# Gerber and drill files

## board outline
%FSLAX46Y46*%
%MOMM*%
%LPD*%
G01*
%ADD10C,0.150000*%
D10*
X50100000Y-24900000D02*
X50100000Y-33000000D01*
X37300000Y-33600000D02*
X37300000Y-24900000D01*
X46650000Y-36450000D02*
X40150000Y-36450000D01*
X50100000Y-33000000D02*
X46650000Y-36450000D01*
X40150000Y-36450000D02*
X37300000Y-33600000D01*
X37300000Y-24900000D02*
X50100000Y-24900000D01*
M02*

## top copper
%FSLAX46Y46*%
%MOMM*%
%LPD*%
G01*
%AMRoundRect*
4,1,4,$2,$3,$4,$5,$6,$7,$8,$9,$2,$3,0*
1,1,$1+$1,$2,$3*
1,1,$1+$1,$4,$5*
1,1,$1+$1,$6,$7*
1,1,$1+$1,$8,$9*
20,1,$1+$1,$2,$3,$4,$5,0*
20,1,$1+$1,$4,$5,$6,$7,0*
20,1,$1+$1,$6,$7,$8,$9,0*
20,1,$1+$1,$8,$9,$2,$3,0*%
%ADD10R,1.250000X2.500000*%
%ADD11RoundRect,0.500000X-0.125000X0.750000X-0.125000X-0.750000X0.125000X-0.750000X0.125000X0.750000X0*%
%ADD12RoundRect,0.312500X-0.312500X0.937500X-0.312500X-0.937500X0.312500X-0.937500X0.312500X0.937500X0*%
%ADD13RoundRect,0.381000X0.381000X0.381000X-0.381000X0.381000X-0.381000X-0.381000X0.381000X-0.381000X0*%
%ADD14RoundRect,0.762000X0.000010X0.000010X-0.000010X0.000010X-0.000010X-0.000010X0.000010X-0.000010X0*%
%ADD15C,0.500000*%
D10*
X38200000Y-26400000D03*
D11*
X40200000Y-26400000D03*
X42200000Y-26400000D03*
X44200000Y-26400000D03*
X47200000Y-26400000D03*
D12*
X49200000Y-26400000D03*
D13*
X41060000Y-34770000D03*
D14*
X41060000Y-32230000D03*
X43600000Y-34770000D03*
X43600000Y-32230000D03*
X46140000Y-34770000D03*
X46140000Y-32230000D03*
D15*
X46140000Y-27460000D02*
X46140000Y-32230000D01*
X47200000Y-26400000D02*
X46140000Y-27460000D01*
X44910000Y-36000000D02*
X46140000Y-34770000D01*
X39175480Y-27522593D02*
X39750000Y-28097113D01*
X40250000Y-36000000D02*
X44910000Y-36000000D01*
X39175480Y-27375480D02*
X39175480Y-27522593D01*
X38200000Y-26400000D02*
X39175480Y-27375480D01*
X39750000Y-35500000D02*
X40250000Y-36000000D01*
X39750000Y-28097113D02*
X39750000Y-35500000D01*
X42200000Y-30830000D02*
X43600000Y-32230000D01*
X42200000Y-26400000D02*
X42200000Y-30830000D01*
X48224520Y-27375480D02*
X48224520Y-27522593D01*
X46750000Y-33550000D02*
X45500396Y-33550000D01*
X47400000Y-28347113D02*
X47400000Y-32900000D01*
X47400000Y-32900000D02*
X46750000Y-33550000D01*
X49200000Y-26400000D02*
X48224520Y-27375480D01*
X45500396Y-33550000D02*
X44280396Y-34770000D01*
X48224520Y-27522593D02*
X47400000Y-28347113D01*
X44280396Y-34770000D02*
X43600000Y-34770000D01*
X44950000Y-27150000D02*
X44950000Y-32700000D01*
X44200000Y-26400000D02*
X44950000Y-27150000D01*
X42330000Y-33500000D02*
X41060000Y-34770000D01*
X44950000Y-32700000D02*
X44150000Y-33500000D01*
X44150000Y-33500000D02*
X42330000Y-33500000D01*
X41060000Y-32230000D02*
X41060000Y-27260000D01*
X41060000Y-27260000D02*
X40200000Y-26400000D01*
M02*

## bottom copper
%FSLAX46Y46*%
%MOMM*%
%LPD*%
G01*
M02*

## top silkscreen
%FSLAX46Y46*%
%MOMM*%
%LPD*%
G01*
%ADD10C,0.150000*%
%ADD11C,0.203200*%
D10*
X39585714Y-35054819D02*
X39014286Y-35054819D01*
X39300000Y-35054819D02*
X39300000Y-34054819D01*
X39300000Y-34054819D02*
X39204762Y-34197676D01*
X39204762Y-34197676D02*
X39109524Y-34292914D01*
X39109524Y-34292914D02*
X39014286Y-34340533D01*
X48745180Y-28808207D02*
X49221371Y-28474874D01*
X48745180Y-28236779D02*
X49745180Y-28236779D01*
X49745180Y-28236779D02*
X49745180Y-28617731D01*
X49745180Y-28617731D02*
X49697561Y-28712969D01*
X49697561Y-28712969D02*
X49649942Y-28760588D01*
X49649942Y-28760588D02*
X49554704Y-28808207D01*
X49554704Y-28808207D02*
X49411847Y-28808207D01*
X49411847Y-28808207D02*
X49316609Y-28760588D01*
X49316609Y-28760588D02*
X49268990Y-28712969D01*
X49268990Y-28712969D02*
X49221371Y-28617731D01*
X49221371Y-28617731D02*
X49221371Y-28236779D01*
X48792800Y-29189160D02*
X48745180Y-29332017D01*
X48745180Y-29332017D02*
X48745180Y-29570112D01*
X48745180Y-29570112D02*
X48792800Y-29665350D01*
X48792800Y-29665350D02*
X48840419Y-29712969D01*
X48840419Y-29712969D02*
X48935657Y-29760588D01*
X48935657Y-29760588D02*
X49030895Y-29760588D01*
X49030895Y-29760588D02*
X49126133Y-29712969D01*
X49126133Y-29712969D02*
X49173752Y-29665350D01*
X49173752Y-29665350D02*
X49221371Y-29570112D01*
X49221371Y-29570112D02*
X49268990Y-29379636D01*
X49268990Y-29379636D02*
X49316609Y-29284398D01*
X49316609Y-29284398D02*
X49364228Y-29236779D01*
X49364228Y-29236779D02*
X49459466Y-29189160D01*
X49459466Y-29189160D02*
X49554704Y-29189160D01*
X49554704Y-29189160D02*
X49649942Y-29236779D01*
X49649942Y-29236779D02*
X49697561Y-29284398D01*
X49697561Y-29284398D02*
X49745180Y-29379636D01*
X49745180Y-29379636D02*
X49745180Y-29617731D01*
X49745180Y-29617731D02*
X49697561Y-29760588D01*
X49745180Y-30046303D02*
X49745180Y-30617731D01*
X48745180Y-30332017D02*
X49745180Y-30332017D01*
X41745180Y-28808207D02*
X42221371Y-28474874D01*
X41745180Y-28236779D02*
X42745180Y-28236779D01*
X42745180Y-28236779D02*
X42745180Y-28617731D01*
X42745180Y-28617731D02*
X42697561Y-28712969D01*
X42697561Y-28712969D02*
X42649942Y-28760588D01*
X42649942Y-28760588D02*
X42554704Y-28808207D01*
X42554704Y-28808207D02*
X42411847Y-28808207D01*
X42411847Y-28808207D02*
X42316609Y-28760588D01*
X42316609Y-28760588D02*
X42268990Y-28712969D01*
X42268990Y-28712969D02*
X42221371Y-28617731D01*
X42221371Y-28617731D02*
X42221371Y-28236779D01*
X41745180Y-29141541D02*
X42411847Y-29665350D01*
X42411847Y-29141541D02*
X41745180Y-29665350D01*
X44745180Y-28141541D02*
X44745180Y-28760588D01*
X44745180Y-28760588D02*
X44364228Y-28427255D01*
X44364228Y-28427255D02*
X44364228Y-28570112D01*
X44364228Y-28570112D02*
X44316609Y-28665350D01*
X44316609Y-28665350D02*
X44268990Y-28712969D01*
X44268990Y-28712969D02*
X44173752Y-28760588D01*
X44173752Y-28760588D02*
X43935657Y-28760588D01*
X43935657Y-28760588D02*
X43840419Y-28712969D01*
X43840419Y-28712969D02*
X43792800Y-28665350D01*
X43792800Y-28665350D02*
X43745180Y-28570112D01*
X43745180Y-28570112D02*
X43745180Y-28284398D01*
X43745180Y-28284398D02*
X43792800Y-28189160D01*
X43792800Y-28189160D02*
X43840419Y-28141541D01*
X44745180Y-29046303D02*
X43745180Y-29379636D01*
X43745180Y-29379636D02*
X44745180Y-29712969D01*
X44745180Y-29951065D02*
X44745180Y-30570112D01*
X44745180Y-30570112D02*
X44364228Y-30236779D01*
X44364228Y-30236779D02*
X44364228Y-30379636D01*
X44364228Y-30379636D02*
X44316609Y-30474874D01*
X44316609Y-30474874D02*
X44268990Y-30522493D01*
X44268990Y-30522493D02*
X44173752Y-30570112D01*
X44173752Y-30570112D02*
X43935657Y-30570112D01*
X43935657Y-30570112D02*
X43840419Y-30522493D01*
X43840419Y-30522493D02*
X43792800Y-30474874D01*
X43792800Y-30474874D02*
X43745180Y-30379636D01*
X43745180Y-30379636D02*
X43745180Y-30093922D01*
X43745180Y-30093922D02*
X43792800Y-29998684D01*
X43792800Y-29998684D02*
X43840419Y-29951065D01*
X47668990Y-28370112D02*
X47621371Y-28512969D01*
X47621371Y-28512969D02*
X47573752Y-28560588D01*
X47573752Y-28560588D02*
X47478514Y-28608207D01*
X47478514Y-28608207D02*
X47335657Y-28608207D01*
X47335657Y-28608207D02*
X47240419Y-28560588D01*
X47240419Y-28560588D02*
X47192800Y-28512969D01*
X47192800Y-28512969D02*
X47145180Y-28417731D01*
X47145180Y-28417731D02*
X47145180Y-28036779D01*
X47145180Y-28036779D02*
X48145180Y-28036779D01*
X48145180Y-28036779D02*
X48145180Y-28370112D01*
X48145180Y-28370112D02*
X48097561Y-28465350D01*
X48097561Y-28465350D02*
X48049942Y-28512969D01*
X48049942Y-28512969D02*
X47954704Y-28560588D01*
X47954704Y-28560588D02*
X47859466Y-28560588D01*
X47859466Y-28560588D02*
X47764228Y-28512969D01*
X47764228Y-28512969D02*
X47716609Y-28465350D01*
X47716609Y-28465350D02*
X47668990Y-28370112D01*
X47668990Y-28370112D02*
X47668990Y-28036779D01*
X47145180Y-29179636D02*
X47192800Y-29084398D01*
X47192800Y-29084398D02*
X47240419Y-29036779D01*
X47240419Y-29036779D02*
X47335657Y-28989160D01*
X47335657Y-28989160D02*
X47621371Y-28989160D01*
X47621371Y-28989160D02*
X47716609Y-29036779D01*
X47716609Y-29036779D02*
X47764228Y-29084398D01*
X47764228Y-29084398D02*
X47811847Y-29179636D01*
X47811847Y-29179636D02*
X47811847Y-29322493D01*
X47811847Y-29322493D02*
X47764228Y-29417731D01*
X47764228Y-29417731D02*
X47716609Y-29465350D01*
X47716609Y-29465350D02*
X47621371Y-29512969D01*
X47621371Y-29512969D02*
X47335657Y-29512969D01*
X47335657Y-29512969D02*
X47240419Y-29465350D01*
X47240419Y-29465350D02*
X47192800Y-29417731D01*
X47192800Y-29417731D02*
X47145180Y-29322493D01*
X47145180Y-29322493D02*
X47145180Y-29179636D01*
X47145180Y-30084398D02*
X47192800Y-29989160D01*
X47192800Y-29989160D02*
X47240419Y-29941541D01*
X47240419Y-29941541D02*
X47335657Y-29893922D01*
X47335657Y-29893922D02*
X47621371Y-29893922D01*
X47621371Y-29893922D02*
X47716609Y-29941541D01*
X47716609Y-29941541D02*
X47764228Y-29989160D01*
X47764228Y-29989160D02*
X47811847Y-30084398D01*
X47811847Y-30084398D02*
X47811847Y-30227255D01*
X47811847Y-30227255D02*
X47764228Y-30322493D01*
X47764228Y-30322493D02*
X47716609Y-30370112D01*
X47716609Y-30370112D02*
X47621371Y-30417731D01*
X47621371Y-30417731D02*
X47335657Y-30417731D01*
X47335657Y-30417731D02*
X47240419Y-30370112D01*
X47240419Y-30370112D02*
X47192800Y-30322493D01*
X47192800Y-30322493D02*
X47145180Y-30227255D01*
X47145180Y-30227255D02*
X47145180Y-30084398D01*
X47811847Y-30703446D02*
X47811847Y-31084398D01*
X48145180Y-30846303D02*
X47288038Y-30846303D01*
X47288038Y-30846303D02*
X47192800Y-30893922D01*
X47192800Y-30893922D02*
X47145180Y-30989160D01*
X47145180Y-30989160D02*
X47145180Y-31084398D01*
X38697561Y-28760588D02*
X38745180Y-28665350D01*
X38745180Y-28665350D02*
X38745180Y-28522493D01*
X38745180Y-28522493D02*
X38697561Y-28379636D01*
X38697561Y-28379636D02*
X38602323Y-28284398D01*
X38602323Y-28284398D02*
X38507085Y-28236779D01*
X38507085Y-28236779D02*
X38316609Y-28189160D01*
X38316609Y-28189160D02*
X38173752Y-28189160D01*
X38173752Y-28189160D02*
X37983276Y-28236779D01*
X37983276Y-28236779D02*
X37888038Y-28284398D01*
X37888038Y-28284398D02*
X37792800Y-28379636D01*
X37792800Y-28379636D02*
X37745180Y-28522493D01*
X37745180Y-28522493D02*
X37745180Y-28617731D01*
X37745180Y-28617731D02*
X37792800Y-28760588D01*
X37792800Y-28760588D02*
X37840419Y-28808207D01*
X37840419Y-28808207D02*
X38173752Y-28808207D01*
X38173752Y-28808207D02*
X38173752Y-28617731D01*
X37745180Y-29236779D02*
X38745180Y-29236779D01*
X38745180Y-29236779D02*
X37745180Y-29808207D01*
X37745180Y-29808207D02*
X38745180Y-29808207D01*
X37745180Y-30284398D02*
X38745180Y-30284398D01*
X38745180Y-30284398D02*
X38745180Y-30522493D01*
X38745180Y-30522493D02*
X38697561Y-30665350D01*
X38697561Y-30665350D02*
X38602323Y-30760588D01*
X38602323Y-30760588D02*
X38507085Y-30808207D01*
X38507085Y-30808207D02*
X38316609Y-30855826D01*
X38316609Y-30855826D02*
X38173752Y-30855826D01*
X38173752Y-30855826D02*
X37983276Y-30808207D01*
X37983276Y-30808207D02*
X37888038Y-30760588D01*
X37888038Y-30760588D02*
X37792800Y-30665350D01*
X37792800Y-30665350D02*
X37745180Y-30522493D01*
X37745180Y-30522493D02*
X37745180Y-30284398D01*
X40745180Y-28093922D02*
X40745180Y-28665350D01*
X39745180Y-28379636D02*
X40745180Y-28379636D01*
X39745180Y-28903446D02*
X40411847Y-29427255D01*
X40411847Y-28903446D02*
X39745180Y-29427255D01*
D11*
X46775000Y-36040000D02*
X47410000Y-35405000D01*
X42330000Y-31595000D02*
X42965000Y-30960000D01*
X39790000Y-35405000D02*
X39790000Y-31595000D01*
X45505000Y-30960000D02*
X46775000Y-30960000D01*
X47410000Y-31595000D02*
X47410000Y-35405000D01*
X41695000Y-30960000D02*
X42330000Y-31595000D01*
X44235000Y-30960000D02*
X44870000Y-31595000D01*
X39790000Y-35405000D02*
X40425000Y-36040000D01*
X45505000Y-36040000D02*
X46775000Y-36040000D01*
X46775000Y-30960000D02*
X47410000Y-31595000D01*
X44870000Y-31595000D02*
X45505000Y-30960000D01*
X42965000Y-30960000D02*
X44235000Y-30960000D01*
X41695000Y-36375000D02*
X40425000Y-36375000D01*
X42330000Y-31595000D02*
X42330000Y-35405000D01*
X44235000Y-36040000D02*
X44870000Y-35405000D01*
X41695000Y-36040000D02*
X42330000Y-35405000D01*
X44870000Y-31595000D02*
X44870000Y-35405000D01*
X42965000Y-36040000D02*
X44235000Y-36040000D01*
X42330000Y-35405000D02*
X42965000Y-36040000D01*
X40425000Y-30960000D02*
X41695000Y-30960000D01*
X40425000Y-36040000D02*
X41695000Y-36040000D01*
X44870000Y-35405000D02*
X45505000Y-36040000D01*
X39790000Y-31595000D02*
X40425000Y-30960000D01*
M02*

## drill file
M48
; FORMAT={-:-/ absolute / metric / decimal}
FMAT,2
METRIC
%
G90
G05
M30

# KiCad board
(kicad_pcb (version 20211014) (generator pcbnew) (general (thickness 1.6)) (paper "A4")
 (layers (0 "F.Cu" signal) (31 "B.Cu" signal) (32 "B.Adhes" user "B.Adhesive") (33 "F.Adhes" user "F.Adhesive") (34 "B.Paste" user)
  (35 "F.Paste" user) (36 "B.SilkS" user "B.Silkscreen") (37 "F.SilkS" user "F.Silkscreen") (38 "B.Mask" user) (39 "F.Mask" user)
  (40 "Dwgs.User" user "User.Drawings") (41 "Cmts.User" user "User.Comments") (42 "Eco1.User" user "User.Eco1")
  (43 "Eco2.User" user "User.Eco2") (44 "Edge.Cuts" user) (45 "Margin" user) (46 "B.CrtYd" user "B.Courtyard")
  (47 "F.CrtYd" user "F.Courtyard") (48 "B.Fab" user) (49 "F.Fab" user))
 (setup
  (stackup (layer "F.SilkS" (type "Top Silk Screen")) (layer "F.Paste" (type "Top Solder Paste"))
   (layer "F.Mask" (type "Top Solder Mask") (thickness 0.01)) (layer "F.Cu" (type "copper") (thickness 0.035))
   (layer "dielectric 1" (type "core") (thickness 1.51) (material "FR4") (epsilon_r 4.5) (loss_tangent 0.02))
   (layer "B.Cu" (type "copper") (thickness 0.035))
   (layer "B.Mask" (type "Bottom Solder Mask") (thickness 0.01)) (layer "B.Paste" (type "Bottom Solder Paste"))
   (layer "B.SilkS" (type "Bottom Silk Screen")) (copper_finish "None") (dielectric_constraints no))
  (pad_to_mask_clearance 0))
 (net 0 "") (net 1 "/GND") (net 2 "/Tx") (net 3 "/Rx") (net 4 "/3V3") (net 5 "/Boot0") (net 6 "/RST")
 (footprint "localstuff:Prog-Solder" (layer "F.Cu") (at 45.7 26.4 -90)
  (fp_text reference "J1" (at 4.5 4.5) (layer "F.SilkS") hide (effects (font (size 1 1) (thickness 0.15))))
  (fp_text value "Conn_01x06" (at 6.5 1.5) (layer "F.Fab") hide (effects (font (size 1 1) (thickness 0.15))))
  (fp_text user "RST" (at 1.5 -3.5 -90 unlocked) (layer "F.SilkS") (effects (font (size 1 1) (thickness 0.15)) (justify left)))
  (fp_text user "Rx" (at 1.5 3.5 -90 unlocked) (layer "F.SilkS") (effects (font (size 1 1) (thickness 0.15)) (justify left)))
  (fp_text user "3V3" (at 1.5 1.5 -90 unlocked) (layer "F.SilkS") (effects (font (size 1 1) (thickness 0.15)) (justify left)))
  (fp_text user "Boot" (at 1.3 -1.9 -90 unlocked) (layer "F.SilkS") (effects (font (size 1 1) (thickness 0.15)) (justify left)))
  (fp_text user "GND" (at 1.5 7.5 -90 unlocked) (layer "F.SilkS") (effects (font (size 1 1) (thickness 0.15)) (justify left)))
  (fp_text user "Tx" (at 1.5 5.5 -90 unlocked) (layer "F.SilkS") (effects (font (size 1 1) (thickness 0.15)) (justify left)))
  (pad "1" smd rect (at 0 7.5 270) (size 2.5 1.25) (layers "F.Cu" "F.Mask") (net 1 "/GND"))
  (pad "2" smd roundrect (at 0 5.5 270) (size 2.5 1.25) (layers "F.Cu" "F.Mask") (roundrect_rratio 0.4) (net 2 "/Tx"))
  (pad "3" smd roundrect (at 0 3.5 270) (size 2.5 1.25) (layers "F.Cu" "F.Mask") (roundrect_rratio 0.4) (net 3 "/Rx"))
  (pad "4" smd roundrect (at 0 1.5 270) (size 2.5 1.25) (layers "F.Cu" "F.Mask") (roundrect_rratio 0.4) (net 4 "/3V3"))
  (pad "5" smd roundrect (at 0 -1.5 270) (size 2.5 1.25) (layers "F.Cu" "F.Mask") (roundrect_rratio 0.4) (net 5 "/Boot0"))
  (pad "6" smd roundrect (at 0 -3.5 270) (size 2.5 1.25) (layers "F.Cu" "F.Mask") (roundrect_rratio 0.25) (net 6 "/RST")))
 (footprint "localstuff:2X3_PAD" (layer "F.Cu") (at 43.6 33.5)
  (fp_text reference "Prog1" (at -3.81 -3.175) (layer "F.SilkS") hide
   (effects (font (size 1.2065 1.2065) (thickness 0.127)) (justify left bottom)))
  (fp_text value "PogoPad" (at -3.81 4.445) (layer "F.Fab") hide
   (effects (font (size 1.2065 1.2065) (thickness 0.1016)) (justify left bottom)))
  (fp_line (start 3.175 2.54) (end 3.81 1.905) (layer "F.SilkS") (width 0.2032))
  (fp_line (start -1.27 -1.905) (end -0.635 -2.54) (layer "F.SilkS") (width 0.2032))
  (fp_line (start -3.81 1.905) (end -3.81 -1.905) (layer "F.SilkS") (width 0.2032))
  (fp_line (start 1.905 -2.54) (end 3.175 -2.54) (layer "F.SilkS") (width 0.2032))
  (fp_line (start 3.81 -1.905) (end 3.81 1.905) (layer "F.SilkS") (width 0.2032))
  (fp_line (start -1.905 -2.54) (end -1.27 -1.905) (layer "F.SilkS") (width 0.2032))
  (fp_line (start 0.635 -2.54) (end 1.27 -1.905) (layer "F.SilkS") (width 0.2032))
  (fp_line (start -3.81 1.905) (end -3.175 2.54) (layer "F.SilkS") (width 0.2032))
  (fp_line (start 1.905 2.54) (end 3.175 2.54) (layer "F.SilkS") (width 0.2032))
  (fp_line (start 3.175 -2.54) (end 3.81 -1.905) (layer "F.SilkS") (width 0.2032))
  (fp_line (start 1.27 -1.905) (end 1.905 -2.54) (layer "F.SilkS") (width 0.2032))
  (fp_line (start -0.635 -2.54) (end 0.635 -2.54) (layer "F.SilkS") (width 0.2032))
  (fp_line (start -1.905 2.875) (end -3.175 2.875) (layer "F.SilkS") (width 0.2032))
  (fp_line (start -1.27 -1.905) (end -1.27 1.905) (layer "F.SilkS") (width 0.2032))
  (fp_line (start 0.635 2.54) (end 1.27 1.905) (layer "F.SilkS") (width 0.2032))
  (fp_line (start -1.905 2.54) (end -1.27 1.905) (layer "F.SilkS") (width 0.2032))
  (fp_line (start 1.27 -1.905) (end 1.27 1.905) (layer "F.SilkS") (width 0.2032))
  (fp_line (start -0.635 2.54) (end 0.635 2.54) (layer "F.SilkS") (width 0.2032))
  (fp_line (start -1.27 1.905) (end -0.635 2.54) (layer "F.SilkS") (width 0.2032))
  (fp_line (start -3.175 -2.54) (end -1.905 -2.54) (layer "F.SilkS") (width 0.2032))
  (fp_line (start -3.175 2.54) (end -1.905 2.54) (layer "F.SilkS") (width 0.2032))
  (fp_line (start 1.27 1.905) (end 1.905 2.54) (layer "F.SilkS") (width 0.2032))
  (fp_line (start -3.81 -1.905) (end -3.175 -2.54) (layer "F.SilkS") (width 0.2032))
  (pad "1" smd roundrect locked (at -2.54 1.27 180) (size 1.524 1.524) (layers "F.Cu" "F.Paste" "F.Mask") (roundrect_rratio 0.25)
   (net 4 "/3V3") (solder_mask_margin 0.1016))
  (pad "2" smd roundrect locked (at -2.54 -1.27 180) (size 1.524 1.524) (layers "F.Cu" "F.Paste" "F.Mask") (roundrect_rratio 0.5)
   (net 2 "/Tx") (solder_mask_margin 0.1016))
  (pad "3" smd roundrect locked (at 0 1.27 180) (size 1.524 1.524) (layers "F.Cu" "F.Paste" "F.Mask") (roundrect_rratio 0.5) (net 6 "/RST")
   (solder_mask_margin 0.1016))
  (pad "4" smd roundrect locked (at 0 -1.27 180) (size 1.524 1.524) (layers "F.Cu" "F.Paste" "F.Mask") (roundrect_rratio 0.5) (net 3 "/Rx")
   (solder_mask_margin 0.1016))
  (pad "5" smd roundrect locked (at 2.54 1.27 180) (size 1.524 1.524) (layers "F.Cu" "F.Paste" "F.Mask") (roundrect_rratio 0.5)
   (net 1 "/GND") (solder_mask_margin 0.1016))
  (pad "6" smd roundrect locked (at 2.54 -1.27 180) (size 1.524 1.524) (layers "F.Cu" "F.Paste" "F.Mask") (roundrect_rratio 0.5)
   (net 5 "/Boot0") (solder_mask_margin 0.1016)))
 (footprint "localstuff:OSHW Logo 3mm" (layer "B.Cu") (at 43.7 29.3 180)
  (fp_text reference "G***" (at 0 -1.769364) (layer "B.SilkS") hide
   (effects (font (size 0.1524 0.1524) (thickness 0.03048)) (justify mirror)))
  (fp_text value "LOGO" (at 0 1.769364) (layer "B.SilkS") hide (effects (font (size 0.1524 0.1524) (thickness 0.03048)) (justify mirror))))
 (gr_line (start 50.1 24.9) (end 50.1 33) (layer "Edge.Cuts") (width 0.15))
 (gr_line (start 37.3 33.6) (end 37.3 24.9) (layer "Edge.Cuts") (width 0.15))
 (gr_line (start 46.65 36.45) (end 40.15 36.45) (layer "Edge.Cuts") (width 0.15))
 (gr_line (start 50.1 33) (end 46.65 36.45) (layer "Edge.Cuts") (width 0.15))
 (gr_line (start 40.15 36.45) (end 37.3 33.6) (layer "Edge.Cuts") (width 0.15))
 (gr_line (start 37.3 24.9) (end 50.1 24.9) (layer "Edge.Cuts") (width 0.15))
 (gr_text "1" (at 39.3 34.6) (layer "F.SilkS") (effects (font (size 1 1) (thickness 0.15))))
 (segment (start 46.14 27.46) (end 46.14 32.23) (width 0.5) (layer "F.Cu") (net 5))
 (segment (start 47.2 26.4) (end 46.14 27.46) (width 0.5) (layer "F.Cu") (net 5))
 (segment (start 44.91 36) (end 46.14 34.77) (width 0.5) (layer "F.Cu") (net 1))
 (segment (start 39.17548 27.522593) (end 39.75 28.097113) (width 0.5) (layer "F.Cu") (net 1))
 (segment (start 40.25 36) (end 44.91 36) (width 0.5) (layer "F.Cu") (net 1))
 (segment (start 39.17548 27.37548) (end 39.17548 27.522593) (width 0.5) (layer "F.Cu") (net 1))
 (segment (start 38.2 26.4) (end 39.17548 27.37548) (width 0.5) (layer "F.Cu") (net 1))
 (segment (start 39.75 35.5) (end 40.25 36) (width 0.5) (layer "F.Cu") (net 1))
 (segment (start 39.75 28.097113) (end 39.75 35.5) (width 0.5) (layer "F.Cu") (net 1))
 (segment (start 42.2 30.83) (end 43.6 32.23) (width 0.5) (layer "F.Cu") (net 3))
 (segment (start 42.2 26.4) (end 42.2 30.83) (width 0.5) (layer "F.Cu") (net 3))
 (segment (start 48.22452 27.37548) (end 48.22452 27.522593) (width 0.5) (layer "F.Cu") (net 6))
 (segment (start 46.75 33.55) (end 45.500396 33.55) (width 0.5) (layer "F.Cu") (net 6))
 (segment (start 47.4 28.347113) (end 47.4 32.9) (width 0.5) (layer "F.Cu") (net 6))
 (segment (start 47.4 32.9) (end 46.75 33.55) (width 0.5) (layer "F.Cu") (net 6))
 (segment (start 49.2 26.4) (end 48.22452 27.37548) (width 0.5) (layer "F.Cu") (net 6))
 (segment (start 45.500396 33.55) (end 44.280396 34.77) (width 0.5) (layer "F.Cu") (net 6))
 (segment (start 48.22452 27.522593) (end 47.4 28.347113) (width 0.5) (layer "F.Cu") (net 6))
 (segment (start 44.280396 34.77) (end 43.6 34.77) (width 0.5) (layer "F.Cu") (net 6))
 (segment (start 44.95 27.15) (end 44.95 32.7) (width 0.5) (layer "F.Cu") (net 4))
 (segment (start 44.2 26.4) (end 44.95 27.15) (width 0.5) (layer "F.Cu") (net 4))
 (segment (start 42.33 33.5) (end 41.06 34.77) (width 0.5) (layer "F.Cu") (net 4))
 (segment (start 44.95 32.7) (end 44.15 33.5) (width 0.5) (layer "F.Cu") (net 4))
 (segment (start 44.15 33.5) (end 42.33 33.5) (width 0.5) (layer "F.Cu") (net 4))
 (segment (start 41.06 32.23) (end 41.06 27.26) (width 0.5) (layer "F.Cu") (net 2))
 (segment (start 41.06 27.26) (end 40.2 26.4) (width 0.5) (layer "F.Cu") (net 2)))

